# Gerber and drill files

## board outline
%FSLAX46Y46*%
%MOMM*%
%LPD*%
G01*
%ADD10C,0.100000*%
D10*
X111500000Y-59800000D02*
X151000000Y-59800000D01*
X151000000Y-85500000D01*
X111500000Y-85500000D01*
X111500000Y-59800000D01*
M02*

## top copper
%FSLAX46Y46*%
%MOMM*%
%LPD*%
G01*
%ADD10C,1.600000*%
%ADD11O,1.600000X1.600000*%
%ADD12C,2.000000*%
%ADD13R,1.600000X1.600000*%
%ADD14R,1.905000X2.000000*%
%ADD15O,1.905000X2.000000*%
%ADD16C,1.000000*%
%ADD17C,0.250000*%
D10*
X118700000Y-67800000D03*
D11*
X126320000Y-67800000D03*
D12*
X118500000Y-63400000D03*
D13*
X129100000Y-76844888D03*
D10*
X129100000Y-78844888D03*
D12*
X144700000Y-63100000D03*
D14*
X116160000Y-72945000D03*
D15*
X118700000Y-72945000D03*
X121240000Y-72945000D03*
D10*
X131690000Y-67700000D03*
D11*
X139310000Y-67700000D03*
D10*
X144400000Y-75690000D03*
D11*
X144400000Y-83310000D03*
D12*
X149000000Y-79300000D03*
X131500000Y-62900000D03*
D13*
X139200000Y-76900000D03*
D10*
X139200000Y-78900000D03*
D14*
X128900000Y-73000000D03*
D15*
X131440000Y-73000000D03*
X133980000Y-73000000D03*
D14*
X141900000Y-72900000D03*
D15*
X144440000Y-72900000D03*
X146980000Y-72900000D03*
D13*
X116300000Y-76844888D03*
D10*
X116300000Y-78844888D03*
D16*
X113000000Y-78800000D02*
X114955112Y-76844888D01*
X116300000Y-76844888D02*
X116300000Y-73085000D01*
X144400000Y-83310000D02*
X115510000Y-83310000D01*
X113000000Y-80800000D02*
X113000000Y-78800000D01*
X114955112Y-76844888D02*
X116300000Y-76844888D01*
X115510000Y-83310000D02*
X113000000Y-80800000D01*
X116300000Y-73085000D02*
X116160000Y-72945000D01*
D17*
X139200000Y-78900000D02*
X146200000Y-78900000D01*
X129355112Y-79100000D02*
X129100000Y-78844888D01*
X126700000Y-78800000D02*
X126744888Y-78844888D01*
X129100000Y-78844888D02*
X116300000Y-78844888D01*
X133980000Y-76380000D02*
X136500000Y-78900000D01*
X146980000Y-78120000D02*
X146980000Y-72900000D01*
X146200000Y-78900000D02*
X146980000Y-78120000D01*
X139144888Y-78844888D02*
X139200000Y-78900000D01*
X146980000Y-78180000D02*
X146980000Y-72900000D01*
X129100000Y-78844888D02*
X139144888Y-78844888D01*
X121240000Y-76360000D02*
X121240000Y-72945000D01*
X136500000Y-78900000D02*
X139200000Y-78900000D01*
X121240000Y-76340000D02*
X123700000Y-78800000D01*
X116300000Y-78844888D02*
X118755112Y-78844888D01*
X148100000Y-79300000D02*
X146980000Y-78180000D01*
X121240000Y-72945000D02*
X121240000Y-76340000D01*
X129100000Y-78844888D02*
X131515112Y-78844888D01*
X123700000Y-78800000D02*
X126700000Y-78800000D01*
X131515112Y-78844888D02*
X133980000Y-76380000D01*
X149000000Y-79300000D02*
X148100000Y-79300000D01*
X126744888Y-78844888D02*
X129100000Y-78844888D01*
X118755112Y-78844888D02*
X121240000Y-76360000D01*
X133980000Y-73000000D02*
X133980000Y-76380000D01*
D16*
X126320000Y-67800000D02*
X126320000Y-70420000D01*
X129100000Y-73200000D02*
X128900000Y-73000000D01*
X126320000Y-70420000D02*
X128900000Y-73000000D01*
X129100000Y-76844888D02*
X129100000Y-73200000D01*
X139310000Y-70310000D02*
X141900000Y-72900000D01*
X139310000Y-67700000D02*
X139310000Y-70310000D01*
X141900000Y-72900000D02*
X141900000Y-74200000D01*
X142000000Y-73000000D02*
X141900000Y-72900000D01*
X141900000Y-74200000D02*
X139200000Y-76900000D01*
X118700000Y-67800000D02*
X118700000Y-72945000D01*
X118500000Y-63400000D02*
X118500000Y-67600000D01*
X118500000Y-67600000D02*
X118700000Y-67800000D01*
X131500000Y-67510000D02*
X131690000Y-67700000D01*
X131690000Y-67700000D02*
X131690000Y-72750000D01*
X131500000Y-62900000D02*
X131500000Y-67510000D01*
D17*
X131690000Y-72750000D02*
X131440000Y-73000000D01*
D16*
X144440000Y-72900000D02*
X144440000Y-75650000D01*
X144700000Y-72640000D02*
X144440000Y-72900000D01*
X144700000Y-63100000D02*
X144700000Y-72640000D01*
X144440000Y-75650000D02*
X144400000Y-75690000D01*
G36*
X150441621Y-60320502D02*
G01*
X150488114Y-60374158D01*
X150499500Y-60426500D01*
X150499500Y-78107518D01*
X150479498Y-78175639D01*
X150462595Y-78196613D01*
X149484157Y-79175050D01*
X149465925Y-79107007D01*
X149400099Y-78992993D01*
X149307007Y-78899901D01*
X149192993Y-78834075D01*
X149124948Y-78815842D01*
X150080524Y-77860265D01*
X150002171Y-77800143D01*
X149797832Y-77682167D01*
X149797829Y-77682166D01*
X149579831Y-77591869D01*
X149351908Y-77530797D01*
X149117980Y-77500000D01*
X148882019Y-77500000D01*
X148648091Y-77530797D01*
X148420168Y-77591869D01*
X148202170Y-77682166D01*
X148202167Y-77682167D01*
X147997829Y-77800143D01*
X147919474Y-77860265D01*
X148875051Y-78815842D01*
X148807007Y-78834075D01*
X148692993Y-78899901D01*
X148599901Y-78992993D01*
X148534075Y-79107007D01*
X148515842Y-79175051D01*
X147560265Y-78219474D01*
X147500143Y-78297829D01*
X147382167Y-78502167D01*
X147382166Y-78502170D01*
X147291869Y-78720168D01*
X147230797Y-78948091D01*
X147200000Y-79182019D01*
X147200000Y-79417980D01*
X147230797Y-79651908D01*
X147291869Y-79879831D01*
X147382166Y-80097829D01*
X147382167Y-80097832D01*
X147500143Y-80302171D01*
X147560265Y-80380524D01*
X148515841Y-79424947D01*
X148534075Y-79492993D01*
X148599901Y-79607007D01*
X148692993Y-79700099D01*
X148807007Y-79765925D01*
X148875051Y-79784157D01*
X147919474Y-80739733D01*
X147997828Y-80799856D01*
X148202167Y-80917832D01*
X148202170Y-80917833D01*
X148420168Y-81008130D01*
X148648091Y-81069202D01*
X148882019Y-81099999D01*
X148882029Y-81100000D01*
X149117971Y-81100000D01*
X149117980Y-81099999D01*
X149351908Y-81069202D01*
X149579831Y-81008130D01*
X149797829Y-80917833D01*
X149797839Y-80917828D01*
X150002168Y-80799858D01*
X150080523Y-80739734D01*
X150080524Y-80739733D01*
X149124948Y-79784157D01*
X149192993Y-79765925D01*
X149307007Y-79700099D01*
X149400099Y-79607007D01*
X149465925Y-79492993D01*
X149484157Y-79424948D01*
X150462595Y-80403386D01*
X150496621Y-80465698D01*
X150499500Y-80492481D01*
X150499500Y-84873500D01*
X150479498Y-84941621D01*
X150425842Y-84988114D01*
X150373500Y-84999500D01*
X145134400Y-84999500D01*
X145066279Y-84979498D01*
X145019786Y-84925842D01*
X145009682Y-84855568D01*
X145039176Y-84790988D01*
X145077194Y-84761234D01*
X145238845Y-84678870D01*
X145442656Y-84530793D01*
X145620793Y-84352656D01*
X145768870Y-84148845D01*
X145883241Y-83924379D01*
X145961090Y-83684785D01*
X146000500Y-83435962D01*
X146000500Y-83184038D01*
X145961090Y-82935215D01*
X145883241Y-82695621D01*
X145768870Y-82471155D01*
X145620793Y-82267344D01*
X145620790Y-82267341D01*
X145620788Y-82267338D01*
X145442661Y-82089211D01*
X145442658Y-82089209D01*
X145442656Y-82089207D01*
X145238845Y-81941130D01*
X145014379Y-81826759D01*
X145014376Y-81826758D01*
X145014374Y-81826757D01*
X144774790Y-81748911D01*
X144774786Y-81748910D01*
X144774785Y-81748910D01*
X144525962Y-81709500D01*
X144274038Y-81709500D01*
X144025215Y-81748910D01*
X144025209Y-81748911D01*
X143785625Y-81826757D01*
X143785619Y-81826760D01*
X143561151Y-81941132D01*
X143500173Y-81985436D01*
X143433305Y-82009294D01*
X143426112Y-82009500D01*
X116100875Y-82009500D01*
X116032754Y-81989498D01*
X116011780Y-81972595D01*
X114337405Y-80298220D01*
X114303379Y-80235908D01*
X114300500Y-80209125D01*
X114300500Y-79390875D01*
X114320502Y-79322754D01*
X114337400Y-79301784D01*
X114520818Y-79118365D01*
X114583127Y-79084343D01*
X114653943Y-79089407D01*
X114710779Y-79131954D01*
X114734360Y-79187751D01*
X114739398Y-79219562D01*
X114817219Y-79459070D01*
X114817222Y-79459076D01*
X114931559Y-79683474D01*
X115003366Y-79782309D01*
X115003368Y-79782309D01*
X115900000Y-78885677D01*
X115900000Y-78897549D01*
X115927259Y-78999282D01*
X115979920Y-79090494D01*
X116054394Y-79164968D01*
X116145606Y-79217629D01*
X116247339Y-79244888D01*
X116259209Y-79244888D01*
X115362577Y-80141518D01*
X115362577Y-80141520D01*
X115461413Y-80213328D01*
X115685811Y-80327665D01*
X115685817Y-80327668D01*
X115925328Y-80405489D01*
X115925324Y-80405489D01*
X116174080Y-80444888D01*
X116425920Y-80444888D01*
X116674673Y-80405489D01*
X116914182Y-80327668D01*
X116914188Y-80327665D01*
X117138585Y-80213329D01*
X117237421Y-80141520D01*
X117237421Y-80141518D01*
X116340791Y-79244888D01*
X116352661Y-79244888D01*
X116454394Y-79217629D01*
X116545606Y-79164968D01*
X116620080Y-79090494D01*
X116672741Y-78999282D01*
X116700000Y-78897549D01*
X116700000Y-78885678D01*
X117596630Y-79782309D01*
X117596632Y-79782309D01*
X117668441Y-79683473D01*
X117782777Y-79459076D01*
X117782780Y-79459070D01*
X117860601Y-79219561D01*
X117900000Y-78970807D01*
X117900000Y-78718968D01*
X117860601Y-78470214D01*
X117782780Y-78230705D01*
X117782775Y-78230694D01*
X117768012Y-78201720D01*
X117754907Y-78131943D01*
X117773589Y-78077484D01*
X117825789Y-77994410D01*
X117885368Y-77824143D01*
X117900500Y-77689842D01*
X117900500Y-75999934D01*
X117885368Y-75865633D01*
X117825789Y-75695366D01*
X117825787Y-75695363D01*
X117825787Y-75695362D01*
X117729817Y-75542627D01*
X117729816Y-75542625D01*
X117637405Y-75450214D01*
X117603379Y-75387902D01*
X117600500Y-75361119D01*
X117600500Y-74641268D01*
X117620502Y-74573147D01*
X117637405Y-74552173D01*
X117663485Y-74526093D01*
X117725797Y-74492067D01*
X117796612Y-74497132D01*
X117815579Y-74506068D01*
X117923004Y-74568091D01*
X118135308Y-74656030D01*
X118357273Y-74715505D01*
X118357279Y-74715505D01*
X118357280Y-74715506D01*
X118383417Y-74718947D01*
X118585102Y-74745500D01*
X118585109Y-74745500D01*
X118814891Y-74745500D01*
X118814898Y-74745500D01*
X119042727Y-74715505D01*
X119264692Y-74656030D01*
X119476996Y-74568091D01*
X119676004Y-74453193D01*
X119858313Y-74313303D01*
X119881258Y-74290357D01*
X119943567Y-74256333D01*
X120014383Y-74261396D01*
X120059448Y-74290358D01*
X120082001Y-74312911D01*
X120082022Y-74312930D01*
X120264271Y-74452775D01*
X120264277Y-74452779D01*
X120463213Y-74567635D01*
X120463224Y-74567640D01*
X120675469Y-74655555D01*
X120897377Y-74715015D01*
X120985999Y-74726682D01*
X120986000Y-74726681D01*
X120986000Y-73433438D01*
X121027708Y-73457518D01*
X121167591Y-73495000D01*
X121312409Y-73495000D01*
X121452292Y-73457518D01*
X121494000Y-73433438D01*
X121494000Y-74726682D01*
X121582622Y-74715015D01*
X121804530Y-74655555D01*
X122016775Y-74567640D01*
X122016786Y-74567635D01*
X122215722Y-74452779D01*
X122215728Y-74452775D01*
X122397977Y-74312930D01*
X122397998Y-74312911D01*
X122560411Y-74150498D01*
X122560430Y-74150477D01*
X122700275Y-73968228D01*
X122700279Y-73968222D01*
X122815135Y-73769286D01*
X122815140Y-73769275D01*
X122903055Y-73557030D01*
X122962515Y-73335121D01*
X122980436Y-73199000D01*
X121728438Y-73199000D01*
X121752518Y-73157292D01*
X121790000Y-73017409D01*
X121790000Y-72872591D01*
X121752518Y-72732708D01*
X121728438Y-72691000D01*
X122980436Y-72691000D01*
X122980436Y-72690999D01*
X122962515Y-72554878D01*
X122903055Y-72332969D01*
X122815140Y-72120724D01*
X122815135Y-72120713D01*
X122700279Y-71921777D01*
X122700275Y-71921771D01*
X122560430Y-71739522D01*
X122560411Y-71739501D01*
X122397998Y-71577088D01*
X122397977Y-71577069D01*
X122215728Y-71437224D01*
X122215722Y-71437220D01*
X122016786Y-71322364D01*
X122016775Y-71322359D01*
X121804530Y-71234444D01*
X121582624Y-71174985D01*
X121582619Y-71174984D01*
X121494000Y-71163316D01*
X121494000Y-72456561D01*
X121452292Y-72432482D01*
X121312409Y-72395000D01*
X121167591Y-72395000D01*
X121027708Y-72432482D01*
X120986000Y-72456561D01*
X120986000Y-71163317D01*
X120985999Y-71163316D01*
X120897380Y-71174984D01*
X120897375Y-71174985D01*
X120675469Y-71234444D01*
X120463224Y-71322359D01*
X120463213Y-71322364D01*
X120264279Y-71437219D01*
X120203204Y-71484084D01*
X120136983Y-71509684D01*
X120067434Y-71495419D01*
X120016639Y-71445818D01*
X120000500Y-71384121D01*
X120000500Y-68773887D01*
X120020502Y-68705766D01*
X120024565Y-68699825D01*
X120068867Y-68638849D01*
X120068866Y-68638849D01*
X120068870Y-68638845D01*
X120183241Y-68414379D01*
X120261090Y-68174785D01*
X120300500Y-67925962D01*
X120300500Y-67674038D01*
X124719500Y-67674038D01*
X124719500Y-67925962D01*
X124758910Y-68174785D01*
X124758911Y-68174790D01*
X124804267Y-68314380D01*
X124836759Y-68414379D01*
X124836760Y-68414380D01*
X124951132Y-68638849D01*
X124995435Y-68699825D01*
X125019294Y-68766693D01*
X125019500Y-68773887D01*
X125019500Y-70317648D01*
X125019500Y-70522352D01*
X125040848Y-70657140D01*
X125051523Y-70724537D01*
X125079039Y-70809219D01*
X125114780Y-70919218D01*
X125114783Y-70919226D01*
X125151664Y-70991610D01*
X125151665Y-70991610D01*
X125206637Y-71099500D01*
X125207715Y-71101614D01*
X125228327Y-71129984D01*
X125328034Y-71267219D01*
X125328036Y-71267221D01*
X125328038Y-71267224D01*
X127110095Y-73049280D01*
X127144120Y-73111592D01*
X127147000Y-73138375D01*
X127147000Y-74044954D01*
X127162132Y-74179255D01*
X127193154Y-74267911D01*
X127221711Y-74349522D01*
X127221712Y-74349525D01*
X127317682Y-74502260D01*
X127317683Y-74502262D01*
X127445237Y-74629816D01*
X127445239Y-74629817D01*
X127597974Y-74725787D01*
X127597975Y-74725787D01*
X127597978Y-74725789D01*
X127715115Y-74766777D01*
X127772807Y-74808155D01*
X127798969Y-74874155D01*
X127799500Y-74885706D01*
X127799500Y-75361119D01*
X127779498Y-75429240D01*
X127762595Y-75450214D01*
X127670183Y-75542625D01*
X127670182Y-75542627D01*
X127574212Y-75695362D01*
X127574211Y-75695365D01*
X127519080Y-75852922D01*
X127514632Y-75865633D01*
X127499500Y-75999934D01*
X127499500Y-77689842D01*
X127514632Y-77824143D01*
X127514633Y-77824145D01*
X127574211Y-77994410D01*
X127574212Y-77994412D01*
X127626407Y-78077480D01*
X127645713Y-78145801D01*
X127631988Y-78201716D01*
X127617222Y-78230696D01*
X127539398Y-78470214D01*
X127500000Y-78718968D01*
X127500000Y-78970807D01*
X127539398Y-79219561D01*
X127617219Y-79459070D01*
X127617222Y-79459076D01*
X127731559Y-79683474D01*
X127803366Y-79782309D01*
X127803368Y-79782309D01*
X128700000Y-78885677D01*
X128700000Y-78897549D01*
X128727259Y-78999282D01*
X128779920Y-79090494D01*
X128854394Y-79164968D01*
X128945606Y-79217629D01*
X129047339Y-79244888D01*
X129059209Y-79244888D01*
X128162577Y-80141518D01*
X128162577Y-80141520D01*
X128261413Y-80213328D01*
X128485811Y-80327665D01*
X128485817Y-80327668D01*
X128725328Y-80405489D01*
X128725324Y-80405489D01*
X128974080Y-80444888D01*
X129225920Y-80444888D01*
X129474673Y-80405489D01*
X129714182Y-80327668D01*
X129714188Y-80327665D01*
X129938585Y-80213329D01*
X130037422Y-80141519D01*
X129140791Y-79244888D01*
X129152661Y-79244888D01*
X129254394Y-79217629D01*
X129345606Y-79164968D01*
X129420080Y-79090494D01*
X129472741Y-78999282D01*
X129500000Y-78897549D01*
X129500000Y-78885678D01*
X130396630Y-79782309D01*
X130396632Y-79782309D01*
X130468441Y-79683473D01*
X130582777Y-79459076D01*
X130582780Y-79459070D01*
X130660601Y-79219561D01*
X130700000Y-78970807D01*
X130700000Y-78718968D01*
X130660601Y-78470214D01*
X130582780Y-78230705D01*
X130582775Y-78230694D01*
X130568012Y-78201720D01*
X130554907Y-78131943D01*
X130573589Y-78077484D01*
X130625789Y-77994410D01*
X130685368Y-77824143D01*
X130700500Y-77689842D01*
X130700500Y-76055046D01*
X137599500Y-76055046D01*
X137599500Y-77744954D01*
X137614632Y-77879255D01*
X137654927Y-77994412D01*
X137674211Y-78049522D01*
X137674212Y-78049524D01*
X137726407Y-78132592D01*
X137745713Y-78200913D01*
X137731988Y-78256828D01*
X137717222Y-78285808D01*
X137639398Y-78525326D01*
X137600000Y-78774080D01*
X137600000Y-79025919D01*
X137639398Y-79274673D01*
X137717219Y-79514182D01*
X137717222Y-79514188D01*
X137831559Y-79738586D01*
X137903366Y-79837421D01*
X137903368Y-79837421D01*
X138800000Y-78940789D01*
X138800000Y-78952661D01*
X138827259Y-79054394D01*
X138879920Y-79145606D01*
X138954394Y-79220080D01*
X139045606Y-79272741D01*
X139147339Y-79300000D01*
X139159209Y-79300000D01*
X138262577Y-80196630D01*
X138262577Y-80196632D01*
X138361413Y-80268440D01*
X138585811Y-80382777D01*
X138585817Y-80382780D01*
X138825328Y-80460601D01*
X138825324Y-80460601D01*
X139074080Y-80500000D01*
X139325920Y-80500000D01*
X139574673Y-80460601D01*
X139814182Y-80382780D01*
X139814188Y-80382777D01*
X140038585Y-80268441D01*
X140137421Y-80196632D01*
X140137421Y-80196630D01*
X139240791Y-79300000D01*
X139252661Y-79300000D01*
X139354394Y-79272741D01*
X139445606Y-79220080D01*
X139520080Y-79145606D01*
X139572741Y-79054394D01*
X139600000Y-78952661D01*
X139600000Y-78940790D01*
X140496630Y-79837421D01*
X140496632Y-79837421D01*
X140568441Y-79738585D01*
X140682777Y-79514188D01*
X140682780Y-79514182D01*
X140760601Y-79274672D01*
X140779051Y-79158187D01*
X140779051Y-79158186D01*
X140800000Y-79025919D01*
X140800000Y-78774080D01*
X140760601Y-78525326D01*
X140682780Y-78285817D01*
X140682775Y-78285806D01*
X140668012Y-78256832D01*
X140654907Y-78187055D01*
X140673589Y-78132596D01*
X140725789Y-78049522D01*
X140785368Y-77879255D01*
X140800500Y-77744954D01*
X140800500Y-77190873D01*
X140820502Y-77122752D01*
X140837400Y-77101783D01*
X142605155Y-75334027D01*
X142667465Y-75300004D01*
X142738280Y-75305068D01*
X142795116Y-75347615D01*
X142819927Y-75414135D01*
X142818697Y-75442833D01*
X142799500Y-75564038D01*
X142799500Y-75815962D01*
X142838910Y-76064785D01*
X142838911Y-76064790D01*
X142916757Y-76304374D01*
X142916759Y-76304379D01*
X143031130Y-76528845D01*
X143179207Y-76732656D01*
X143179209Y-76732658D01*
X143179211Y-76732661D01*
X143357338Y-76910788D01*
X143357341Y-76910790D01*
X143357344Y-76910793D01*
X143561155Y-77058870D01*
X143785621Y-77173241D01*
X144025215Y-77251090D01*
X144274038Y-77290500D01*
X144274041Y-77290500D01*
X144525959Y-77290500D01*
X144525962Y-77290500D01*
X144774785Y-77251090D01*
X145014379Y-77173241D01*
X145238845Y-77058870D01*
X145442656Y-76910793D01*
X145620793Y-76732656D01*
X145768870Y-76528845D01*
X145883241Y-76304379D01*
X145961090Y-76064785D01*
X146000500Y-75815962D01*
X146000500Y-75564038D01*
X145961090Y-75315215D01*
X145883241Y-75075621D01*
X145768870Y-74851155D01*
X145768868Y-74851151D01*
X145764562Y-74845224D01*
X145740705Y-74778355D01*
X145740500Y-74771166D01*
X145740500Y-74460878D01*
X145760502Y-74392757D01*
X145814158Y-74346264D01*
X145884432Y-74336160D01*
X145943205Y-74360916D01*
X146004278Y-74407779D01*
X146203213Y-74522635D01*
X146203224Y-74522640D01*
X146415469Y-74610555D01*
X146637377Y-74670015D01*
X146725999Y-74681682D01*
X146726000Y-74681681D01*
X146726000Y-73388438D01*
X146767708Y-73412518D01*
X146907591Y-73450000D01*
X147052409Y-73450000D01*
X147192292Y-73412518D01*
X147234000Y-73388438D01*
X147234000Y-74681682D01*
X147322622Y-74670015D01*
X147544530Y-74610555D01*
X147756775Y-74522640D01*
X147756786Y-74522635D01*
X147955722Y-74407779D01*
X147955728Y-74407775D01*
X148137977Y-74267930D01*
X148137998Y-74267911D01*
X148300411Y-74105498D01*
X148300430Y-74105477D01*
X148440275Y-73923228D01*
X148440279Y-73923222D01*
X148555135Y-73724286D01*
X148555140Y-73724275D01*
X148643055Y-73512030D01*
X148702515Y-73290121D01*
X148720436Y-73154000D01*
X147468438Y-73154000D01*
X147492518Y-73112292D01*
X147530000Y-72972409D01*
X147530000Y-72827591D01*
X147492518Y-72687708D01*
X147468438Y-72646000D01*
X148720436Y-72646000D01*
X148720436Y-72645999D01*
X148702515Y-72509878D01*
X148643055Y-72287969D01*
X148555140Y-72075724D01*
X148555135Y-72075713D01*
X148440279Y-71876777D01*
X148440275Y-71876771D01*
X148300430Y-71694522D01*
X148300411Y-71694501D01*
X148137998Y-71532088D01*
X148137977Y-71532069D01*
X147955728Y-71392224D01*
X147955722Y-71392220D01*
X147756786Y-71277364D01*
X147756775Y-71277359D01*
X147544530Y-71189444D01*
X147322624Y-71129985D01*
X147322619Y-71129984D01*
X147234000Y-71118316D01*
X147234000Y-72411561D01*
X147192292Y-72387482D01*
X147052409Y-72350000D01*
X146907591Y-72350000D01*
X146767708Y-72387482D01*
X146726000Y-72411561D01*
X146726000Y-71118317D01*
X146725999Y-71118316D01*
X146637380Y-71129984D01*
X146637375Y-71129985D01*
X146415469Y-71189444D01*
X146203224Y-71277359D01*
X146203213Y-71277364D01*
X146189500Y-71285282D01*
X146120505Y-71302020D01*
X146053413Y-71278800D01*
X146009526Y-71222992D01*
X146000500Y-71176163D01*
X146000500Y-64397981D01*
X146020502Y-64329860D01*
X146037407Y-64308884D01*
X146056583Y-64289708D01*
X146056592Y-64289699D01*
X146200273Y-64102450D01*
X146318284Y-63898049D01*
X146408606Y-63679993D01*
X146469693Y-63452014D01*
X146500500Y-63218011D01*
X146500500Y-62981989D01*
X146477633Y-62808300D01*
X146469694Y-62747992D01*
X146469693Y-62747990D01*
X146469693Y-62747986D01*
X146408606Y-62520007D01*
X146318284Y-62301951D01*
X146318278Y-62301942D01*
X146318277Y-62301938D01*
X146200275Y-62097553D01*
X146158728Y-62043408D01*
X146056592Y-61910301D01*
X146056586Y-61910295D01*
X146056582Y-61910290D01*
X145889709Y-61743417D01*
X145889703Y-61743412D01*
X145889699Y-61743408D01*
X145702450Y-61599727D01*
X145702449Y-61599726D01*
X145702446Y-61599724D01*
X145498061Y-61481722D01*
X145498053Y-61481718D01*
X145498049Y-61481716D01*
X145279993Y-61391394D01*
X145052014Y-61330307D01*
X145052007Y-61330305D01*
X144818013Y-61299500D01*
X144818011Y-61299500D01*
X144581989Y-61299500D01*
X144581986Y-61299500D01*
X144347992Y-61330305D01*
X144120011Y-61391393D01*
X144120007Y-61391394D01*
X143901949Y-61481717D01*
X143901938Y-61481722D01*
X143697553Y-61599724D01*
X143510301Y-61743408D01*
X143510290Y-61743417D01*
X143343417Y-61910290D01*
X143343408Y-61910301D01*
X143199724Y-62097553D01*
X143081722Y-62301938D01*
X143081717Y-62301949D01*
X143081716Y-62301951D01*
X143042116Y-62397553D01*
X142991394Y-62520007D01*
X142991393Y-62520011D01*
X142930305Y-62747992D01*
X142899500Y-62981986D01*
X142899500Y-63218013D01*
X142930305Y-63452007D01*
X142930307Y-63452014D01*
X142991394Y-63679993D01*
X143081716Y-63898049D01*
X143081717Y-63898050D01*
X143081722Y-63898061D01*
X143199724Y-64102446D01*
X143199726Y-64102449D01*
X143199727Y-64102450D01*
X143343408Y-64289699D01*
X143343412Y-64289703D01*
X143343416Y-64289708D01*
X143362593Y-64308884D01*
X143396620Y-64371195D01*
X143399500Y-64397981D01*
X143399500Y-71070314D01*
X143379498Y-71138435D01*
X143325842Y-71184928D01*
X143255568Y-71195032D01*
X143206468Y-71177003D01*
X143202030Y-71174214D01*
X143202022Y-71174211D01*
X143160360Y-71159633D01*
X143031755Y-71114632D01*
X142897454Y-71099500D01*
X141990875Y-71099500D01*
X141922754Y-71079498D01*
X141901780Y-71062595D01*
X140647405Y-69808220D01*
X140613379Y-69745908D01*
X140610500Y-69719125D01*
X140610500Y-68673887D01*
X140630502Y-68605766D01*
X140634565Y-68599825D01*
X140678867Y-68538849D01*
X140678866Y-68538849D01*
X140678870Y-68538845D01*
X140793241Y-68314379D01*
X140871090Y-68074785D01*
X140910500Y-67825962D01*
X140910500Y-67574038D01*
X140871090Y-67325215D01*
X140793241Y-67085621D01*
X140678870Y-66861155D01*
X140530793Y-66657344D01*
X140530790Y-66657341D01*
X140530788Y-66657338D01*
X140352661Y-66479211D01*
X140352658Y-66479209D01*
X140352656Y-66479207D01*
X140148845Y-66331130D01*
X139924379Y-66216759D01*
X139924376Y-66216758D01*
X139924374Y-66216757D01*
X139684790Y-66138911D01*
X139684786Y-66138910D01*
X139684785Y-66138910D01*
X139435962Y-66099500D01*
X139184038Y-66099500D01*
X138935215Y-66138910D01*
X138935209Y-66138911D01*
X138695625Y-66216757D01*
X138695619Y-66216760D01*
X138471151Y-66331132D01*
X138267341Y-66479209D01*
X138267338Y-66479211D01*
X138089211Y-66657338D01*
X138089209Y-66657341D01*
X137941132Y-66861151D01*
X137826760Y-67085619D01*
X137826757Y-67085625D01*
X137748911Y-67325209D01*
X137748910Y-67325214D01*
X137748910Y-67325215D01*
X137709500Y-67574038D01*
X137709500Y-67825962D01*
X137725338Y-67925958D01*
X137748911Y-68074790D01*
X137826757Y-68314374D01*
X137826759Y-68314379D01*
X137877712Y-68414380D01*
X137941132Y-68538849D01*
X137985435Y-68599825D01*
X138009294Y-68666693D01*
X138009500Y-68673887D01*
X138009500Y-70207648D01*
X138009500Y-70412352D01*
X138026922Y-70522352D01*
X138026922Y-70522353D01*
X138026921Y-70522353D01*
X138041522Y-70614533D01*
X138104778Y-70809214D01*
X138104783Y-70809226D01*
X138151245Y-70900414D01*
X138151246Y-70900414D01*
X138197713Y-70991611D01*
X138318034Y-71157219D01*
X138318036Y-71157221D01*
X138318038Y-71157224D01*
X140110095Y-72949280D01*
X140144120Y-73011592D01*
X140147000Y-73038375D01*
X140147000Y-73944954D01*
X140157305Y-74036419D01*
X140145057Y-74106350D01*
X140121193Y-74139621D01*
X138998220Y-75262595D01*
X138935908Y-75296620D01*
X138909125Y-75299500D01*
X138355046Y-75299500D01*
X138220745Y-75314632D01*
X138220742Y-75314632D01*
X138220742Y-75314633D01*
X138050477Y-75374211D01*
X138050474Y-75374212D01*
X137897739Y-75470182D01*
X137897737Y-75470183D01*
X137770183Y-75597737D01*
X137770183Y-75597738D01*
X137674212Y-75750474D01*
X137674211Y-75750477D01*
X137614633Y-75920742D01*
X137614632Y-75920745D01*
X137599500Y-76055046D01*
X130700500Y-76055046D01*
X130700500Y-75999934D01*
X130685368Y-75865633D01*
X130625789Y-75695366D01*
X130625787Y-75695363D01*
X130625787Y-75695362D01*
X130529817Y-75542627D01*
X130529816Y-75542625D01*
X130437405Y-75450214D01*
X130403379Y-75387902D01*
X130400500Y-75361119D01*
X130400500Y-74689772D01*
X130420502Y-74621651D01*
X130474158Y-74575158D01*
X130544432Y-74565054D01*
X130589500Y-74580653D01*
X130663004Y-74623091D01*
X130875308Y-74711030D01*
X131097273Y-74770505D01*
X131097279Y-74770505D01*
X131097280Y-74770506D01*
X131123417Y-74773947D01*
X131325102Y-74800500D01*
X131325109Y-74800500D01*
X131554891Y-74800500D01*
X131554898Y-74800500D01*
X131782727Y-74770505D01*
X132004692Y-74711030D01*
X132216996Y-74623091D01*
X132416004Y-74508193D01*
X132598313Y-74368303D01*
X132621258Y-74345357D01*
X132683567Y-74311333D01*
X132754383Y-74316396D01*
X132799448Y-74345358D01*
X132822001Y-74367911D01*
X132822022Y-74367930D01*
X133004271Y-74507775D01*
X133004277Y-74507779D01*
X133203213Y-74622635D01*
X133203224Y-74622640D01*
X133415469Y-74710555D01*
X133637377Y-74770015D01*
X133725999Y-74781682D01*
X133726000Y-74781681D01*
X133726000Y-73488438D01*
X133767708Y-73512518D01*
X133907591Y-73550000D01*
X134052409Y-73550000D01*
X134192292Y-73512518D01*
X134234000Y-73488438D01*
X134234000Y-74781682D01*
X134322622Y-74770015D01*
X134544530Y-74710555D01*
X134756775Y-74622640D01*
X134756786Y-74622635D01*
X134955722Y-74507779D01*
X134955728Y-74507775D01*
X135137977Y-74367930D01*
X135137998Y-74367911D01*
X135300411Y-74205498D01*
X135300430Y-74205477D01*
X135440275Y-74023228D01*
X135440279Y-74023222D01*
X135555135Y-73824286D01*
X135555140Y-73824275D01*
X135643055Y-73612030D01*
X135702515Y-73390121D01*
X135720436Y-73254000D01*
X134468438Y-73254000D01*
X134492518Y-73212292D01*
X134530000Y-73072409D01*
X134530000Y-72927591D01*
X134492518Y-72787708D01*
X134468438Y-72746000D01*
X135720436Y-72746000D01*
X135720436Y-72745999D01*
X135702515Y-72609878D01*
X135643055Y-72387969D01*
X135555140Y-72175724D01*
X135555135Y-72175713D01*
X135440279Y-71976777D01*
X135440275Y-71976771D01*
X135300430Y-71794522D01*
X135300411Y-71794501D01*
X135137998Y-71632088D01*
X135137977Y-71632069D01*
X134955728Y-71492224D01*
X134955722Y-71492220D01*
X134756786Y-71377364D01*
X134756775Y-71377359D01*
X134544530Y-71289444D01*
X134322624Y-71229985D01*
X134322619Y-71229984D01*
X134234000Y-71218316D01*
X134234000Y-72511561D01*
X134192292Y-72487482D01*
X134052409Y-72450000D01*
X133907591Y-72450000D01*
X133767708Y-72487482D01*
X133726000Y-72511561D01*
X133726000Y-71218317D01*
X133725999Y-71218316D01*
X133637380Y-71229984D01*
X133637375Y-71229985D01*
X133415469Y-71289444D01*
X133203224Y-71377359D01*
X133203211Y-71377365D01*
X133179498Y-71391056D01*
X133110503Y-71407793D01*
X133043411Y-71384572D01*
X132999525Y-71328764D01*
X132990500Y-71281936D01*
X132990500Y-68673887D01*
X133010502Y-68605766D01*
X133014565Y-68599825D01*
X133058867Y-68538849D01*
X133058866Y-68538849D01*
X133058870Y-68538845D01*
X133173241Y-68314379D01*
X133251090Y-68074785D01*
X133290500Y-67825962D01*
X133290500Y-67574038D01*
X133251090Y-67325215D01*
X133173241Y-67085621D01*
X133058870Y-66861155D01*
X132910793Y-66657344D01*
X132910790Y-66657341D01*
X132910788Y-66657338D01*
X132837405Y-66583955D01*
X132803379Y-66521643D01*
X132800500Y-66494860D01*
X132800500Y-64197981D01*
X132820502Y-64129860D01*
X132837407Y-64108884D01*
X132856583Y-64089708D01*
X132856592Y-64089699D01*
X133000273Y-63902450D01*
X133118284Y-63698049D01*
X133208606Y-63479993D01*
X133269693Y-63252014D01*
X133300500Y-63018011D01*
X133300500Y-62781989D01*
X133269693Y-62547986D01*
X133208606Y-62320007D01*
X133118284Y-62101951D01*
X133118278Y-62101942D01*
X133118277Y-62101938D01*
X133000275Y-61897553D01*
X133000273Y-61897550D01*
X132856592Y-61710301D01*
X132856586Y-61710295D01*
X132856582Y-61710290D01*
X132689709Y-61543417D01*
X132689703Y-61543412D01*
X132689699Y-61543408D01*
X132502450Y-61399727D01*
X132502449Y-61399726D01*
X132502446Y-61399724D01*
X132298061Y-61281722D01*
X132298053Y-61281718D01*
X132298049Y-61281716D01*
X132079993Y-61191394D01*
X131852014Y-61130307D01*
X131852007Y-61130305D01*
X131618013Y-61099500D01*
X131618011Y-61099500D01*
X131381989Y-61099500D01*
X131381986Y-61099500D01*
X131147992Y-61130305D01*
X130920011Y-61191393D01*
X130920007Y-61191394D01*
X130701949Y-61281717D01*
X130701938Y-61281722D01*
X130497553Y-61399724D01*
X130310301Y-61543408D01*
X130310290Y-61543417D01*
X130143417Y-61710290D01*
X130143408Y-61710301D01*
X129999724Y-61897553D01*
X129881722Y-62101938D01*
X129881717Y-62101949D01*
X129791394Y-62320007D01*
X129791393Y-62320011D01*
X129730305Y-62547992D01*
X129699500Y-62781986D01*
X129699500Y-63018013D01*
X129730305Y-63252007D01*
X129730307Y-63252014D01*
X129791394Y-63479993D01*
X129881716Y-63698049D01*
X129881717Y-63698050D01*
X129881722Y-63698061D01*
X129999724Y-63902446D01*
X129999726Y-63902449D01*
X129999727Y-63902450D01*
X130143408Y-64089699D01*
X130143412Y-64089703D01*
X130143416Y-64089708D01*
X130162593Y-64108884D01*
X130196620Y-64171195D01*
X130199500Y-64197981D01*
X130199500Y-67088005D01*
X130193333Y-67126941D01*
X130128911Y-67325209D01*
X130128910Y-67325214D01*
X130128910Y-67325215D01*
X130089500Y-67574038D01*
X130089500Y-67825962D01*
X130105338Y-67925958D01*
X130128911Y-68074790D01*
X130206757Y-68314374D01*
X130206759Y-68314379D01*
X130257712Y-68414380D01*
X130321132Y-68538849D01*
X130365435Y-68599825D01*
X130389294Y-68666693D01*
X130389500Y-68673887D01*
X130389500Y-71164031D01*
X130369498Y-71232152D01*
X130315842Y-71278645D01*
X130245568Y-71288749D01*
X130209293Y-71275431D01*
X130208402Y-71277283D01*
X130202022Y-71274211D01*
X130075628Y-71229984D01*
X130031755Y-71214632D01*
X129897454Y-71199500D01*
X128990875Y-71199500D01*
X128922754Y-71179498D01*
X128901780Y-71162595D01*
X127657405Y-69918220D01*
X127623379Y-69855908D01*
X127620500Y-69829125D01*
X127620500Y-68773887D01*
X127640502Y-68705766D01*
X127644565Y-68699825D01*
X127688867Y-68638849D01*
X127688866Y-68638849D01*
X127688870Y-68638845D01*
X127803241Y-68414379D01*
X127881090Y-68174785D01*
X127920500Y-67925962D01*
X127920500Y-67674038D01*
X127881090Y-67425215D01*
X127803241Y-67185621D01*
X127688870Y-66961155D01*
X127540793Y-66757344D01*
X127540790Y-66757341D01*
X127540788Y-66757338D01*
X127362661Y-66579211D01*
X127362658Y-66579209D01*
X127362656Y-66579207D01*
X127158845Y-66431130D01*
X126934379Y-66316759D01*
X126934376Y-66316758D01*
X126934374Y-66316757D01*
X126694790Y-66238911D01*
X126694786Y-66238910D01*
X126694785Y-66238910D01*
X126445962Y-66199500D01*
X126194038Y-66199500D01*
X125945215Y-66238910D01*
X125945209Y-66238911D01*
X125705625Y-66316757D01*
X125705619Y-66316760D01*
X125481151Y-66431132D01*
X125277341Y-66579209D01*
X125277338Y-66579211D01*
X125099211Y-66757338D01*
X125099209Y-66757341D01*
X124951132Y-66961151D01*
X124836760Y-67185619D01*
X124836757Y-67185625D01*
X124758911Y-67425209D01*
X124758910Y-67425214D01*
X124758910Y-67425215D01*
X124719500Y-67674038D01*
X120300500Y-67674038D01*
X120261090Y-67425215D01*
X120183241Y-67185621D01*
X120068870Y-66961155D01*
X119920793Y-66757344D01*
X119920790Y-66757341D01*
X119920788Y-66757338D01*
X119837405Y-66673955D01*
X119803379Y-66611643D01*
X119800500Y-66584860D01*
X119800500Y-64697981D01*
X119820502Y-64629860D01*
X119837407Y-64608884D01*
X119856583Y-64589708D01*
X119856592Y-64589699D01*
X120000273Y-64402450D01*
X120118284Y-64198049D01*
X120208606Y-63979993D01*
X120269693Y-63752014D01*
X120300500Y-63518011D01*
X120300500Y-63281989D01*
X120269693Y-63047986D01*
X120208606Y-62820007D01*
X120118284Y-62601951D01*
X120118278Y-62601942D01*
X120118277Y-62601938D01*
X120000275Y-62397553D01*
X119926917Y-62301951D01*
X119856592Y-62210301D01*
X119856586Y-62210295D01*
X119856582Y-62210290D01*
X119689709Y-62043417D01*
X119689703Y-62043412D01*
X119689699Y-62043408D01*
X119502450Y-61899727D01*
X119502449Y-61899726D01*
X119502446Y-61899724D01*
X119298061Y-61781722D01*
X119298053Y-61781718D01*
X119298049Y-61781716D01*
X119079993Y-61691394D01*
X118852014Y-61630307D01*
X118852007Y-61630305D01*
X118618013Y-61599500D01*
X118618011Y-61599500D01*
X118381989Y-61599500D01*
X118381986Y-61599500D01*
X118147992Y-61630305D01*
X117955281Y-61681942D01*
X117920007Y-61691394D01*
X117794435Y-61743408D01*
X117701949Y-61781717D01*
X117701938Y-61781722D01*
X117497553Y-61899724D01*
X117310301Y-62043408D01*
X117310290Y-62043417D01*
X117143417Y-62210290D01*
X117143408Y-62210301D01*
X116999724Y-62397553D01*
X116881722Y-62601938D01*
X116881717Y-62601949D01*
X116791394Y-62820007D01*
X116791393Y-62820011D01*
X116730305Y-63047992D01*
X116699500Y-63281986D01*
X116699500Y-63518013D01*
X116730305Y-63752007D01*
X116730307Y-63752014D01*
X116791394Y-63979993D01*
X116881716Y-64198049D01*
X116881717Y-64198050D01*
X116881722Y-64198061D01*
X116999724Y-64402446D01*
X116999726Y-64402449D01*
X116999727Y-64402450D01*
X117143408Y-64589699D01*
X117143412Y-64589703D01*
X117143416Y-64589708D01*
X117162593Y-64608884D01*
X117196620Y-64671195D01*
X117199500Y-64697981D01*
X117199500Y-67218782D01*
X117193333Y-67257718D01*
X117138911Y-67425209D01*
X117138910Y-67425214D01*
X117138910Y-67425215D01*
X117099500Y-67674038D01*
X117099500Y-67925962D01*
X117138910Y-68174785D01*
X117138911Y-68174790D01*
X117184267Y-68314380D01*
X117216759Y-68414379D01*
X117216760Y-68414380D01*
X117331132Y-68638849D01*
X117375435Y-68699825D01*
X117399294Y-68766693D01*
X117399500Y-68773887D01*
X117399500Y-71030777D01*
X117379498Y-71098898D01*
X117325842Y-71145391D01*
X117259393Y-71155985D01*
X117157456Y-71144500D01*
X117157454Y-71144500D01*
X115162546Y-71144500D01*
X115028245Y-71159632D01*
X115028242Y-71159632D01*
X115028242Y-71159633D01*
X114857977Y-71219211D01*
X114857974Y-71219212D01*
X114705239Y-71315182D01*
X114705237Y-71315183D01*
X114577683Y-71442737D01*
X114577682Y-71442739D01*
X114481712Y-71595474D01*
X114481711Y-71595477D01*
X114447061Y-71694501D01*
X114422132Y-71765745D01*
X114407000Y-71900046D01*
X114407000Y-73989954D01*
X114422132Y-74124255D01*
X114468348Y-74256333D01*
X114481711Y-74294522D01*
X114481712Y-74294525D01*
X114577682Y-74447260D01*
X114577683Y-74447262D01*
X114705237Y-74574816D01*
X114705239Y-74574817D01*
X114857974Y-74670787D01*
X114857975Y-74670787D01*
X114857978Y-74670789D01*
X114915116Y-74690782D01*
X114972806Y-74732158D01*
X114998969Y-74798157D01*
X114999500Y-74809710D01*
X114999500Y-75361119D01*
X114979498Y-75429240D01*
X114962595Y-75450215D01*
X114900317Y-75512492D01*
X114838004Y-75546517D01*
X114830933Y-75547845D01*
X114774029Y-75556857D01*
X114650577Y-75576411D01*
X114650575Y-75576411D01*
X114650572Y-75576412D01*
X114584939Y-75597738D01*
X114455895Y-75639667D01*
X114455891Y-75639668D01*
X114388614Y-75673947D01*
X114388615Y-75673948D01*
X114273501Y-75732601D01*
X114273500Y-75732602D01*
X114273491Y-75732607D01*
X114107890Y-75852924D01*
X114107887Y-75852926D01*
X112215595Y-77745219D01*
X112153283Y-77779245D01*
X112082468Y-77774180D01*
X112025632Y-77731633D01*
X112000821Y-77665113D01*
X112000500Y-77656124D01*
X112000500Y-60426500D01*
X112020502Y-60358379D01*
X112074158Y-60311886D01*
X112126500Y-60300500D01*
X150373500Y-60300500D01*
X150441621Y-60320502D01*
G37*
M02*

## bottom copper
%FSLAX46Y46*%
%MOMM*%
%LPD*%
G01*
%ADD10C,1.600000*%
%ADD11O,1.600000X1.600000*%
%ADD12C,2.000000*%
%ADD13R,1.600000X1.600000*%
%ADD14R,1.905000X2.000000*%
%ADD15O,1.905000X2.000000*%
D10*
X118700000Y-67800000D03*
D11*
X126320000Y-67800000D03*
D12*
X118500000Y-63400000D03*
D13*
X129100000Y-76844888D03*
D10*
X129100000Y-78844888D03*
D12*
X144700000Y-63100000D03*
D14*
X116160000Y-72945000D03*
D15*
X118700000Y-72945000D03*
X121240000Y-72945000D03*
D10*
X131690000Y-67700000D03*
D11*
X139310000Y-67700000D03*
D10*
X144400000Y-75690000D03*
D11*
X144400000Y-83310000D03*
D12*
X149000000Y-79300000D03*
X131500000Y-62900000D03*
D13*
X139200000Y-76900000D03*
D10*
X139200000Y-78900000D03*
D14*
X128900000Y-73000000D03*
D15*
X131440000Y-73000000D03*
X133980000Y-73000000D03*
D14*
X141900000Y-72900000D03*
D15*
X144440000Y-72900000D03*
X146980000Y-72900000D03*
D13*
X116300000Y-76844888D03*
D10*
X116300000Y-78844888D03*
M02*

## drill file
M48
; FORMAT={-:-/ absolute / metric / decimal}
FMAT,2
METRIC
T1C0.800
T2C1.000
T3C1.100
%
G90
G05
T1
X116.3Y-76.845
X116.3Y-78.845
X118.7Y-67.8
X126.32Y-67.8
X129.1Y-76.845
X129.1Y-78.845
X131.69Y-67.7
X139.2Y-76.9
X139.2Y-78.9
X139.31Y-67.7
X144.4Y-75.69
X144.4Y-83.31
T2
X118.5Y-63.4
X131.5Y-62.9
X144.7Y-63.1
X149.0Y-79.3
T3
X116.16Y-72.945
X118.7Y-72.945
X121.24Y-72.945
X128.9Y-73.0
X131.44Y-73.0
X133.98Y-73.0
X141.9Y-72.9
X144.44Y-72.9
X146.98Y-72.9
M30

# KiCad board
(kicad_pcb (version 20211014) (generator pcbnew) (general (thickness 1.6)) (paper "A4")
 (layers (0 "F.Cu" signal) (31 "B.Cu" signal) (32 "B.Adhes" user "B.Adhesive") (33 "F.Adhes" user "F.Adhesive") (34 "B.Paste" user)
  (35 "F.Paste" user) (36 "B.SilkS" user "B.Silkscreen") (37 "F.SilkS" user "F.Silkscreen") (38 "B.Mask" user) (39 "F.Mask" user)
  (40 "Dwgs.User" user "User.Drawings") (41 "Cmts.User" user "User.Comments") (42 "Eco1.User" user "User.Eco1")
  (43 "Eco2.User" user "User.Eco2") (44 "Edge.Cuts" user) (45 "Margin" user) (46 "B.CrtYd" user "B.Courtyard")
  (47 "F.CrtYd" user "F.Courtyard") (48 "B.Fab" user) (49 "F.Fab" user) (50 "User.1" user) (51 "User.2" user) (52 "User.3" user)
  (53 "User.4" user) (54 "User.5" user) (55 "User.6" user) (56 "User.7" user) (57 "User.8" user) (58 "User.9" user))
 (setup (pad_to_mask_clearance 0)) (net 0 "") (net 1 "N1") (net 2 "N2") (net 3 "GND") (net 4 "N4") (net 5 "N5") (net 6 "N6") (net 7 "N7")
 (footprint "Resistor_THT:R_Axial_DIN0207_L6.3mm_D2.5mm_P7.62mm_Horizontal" (layer "F.Cu") (at 118.7 67.8)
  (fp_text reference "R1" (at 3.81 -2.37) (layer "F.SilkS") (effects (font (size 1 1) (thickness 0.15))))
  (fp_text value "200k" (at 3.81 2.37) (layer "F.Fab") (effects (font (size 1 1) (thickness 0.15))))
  (pad "1" thru_hole circle (at 0 0) (size 1.6 1.6) (drill 0.8) (layers *.Cu *.Mask) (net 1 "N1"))
  (pad "2" thru_hole oval (at 7.62 0) (size 1.6 1.6) (drill 0.8) (layers *.Cu *.Mask) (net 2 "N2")))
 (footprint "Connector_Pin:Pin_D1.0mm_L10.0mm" (layer "F.Cu") (at 118.5 63.4)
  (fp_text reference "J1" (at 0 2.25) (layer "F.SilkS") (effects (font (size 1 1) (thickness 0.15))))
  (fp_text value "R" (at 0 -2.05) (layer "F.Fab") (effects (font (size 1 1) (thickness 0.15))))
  (pad "1" thru_hole circle (at 0 0) (size 2 2) (drill 1) (layers *.Cu *.Mask) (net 1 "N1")))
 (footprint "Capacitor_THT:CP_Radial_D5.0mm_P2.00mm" (layer "F.Cu") (at 129.1 76.844888 -90)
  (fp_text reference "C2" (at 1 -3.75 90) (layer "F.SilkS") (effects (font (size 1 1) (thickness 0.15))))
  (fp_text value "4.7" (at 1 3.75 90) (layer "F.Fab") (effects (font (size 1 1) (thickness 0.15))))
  (pad "1" thru_hole rect (at 0 0 270) (size 1.6 1.6) (drill 0.8) (layers *.Cu *.Mask) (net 2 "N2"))
  (pad "2" thru_hole circle (at 2 0 270) (size 1.6 1.6) (drill 0.8) (layers *.Cu *.Mask) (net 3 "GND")))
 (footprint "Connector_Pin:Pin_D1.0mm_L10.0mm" (layer "F.Cu") (at 144.7 63.1)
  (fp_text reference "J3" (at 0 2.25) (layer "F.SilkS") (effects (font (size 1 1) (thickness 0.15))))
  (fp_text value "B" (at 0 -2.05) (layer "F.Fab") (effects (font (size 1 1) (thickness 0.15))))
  (pad "1" thru_hole circle (at 0 0) (size 2 2) (drill 1) (layers *.Cu *.Mask) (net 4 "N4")))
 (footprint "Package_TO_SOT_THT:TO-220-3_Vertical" (layer "F.Cu") (at 116.16 72.945)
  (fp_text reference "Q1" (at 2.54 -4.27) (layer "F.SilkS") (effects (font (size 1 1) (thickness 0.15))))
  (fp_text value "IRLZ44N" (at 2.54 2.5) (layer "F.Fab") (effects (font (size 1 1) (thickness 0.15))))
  (pad "1" thru_hole rect (at 0 0) (size 1.905 2) (drill 1.1) (layers *.Cu *.Mask) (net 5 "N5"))
  (pad "2" thru_hole oval (at 2.54 0) (size 1.905 2) (drill 1.1) (layers *.Cu *.Mask) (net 1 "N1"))
  (pad "3" thru_hole oval (at 5.08 0) (size 1.905 2) (drill 1.1) (layers *.Cu *.Mask) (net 3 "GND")))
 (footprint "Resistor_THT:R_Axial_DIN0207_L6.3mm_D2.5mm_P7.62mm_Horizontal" (layer "F.Cu") (at 131.69 67.7)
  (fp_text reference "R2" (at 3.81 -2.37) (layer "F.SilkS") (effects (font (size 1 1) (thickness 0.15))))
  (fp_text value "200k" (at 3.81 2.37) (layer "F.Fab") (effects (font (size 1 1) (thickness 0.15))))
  (pad "1" thru_hole circle (at 0 0) (size 1.6 1.6) (drill 0.8) (layers *.Cu *.Mask) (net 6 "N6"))
  (pad "2" thru_hole oval (at 7.62 0) (size 1.6 1.6) (drill 0.8) (layers *.Cu *.Mask) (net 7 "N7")))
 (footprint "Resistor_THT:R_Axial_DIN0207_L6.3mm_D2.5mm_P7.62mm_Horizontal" (layer "F.Cu") (at 144.4 75.69 -90)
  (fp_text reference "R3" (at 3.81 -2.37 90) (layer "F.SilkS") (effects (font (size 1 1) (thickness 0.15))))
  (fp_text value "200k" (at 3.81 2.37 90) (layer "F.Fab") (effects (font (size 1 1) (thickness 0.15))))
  (pad "1" thru_hole circle (at 0 0 270) (size 1.6 1.6) (drill 0.8) (layers *.Cu *.Mask) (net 4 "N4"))
  (pad "2" thru_hole oval (at 7.62 0 270) (size 1.6 1.6) (drill 0.8) (layers *.Cu *.Mask) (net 5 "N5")))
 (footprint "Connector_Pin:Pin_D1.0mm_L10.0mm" (layer "F.Cu") (at 149 79.3)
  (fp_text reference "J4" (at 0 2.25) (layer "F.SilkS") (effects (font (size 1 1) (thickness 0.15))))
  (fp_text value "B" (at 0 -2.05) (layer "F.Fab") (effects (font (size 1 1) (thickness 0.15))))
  (pad "1" thru_hole circle (at 0 0) (size 2 2) (drill 1) (layers *.Cu *.Mask) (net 3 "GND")))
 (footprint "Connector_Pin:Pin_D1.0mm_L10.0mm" (layer "F.Cu") (at 131.5 62.9)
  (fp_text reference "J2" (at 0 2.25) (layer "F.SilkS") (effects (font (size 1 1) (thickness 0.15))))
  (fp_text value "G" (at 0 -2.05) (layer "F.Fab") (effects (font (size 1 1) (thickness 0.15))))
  (pad "1" thru_hole circle (at 0 0) (size 2 2) (drill 1) (layers *.Cu *.Mask) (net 6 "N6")))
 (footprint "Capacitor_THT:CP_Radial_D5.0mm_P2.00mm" (layer "F.Cu") (at 139.2 76.9 -90)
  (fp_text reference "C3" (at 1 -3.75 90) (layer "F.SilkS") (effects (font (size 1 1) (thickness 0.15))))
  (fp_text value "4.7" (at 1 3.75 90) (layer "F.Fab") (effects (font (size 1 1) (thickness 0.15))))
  (pad "1" thru_hole rect (at 0 0 270) (size 1.6 1.6) (drill 0.8) (layers *.Cu *.Mask) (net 7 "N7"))
  (pad "2" thru_hole circle (at 2 0 270) (size 1.6 1.6) (drill 0.8) (layers *.Cu *.Mask) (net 3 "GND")))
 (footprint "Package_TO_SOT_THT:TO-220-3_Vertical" (layer "F.Cu") (at 128.9 73)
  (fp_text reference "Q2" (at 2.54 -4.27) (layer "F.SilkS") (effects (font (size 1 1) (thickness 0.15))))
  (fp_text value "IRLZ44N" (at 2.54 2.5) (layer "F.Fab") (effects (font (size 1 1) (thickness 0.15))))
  (pad "1" thru_hole rect (at 0 0) (size 1.905 2) (drill 1.1) (layers *.Cu *.Mask) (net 2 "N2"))
  (pad "2" thru_hole oval (at 2.54 0) (size 1.905 2) (drill 1.1) (layers *.Cu *.Mask) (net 6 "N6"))
  (pad "3" thru_hole oval (at 5.08 0) (size 1.905 2) (drill 1.1) (layers *.Cu *.Mask) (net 3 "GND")))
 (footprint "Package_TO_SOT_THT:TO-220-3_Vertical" (layer "F.Cu") (at 141.9 72.9)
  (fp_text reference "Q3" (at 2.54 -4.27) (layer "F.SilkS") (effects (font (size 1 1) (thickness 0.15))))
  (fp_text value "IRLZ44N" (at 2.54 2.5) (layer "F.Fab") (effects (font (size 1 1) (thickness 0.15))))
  (pad "1" thru_hole rect (at 0 0) (size 1.905 2) (drill 1.1) (layers *.Cu *.Mask) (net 7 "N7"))
  (pad "2" thru_hole oval (at 2.54 0) (size 1.905 2) (drill 1.1) (layers *.Cu *.Mask) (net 4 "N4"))
  (pad "3" thru_hole oval (at 5.08 0) (size 1.905 2) (drill 1.1) (layers *.Cu *.Mask) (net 3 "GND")))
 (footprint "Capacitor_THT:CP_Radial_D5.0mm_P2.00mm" (layer "F.Cu") (at 116.3 76.844888 -90)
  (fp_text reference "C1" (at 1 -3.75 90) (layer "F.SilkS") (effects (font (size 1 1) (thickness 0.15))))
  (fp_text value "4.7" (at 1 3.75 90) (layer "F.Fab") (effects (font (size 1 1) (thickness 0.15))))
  (pad "1" thru_hole rect (at 0 0 270) (size 1.6 1.6) (drill 0.8) (layers *.Cu *.Mask) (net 5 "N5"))
  (pad "2" thru_hole circle (at 2 0 270) (size 1.6 1.6) (drill 0.8) (layers *.Cu *.Mask) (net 3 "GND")))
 (gr_rect (start 151 85.5) (end 111.5 59.8) (layer "Edge.Cuts") (width 0.1) (fill none))
 (segment (start 113 78.8) (end 114.955112 76.844888) (width 1) (layer "F.Cu") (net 5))
 (segment (start 116.3 76.844888) (end 116.3 73.085) (width 1) (layer "F.Cu") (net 5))
 (segment (start 144.4 83.31) (end 115.51 83.31) (width 1) (layer "F.Cu") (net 5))
 (segment (start 113 80.8) (end 113 78.8) (width 1) (layer "F.Cu") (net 5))
 (segment (start 114.955112 76.844888) (end 116.3 76.844888) (width 1) (layer "F.Cu") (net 5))
 (segment (start 115.51 83.31) (end 113 80.8) (width 1) (layer "F.Cu") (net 5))
 (segment (start 116.3 73.085) (end 116.16 72.945) (width 1) (layer "F.Cu") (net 5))
 (segment (start 139.2 78.9) (end 146.2 78.9) (width 0.25) (layer "F.Cu") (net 3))
 (segment (start 129.355112 79.1) (end 129.1 78.844888) (width 0.25) (layer "F.Cu") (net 3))
 (segment (start 126.7 78.8) (end 126.744888 78.844888) (width 0.25) (layer "F.Cu") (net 3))
 (segment (start 129.1 78.844888) (end 116.3 78.844888) (width 0.25) (layer "F.Cu") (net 3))
 (segment (start 133.98 76.38) (end 136.5 78.9) (width 0.25) (layer "F.Cu") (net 3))
 (segment (start 146.98 78.12) (end 146.98 72.9) (width 0.25) (layer "F.Cu") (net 3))
 (segment (start 146.2 78.9) (end 146.98 78.12) (width 0.25) (layer "F.Cu") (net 3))
 (segment (start 139.144888 78.844888) (end 139.2 78.9) (width 0.25) (layer "F.Cu") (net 3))
 (segment (start 146.98 78.18) (end 146.98 72.9) (width 0.25) (layer "F.Cu") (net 3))
 (segment (start 129.1 78.844888) (end 139.144888 78.844888) (width 0.25) (layer "F.Cu") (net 3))
 (segment (start 121.24 76.36) (end 121.24 72.945) (width 0.25) (layer "F.Cu") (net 3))
 (segment (start 136.5 78.9) (end 139.2 78.9) (width 0.25) (layer "F.Cu") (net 3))
 (segment (start 121.24 76.34) (end 123.7 78.8) (width 0.25) (layer "F.Cu") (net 3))
 (segment (start 116.3 78.844888) (end 118.755112 78.844888) (width 0.25) (layer "F.Cu") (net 3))
 (segment (start 148.1 79.3) (end 146.98 78.18) (width 0.25) (layer "F.Cu") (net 3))
 (segment (start 121.24 72.945) (end 121.24 76.34) (width 0.25) (layer "F.Cu") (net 3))
 (segment (start 129.1 78.844888) (end 131.515112 78.844888) (width 0.25) (layer "F.Cu") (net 3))
 (segment (start 123.7 78.8) (end 126.7 78.8) (width 0.25) (layer "F.Cu") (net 3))
 (segment (start 131.515112 78.844888) (end 133.98 76.38) (width 0.25) (layer "F.Cu") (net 3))
 (segment (start 149 79.3) (end 148.1 79.3) (width 0.25) (layer "F.Cu") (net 3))
 (segment (start 126.744888 78.844888) (end 129.1 78.844888) (width 0.25) (layer "F.Cu") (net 3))
 (segment (start 118.755112 78.844888) (end 121.24 76.36) (width 0.25) (layer "F.Cu") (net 3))
 (segment (start 133.98 73) (end 133.98 76.38) (width 0.25) (layer "F.Cu") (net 3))
 (segment (start 126.32 67.8) (end 126.32 70.42) (width 1) (layer "F.Cu") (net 2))
 (segment (start 129.1 73.2) (end 128.9 73) (width 1) (layer "F.Cu") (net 2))
 (segment (start 126.32 70.42) (end 128.9 73) (width 1) (layer "F.Cu") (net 2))
 (segment (start 129.1 76.844888) (end 129.1 73.2) (width 1) (layer "F.Cu") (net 2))
 (segment (start 139.31 70.31) (end 141.9 72.9) (width 1) (layer "F.Cu") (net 7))
 (segment (start 139.31 67.7) (end 139.31 70.31) (width 1) (layer "F.Cu") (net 7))
 (segment (start 141.9 72.9) (end 141.9 74.2) (width 1) (layer "F.Cu") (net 7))
 (segment (start 142 73) (end 141.9 72.9) (width 1) (layer "F.Cu") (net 7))
 (segment (start 141.9 74.2) (end 139.2 76.9) (width 1) (layer "F.Cu") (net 7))
 (segment (start 118.7 67.8) (end 118.7 72.945) (width 1) (layer "F.Cu") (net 1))
 (segment (start 118.5 63.4) (end 118.5 67.6) (width 1) (layer "F.Cu") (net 1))
 (segment (start 118.5 67.6) (end 118.7 67.8) (width 1) (layer "F.Cu") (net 1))
 (segment (start 131.5 67.51) (end 131.69 67.7) (width 1) (layer "F.Cu") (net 6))
 (segment (start 131.69 67.7) (end 131.69 72.75) (width 1) (layer "F.Cu") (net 6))
 (segment (start 131.5 62.9) (end 131.5 67.51) (width 1) (layer "F.Cu") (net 6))
 (segment (start 131.69 72.75) (end 131.44 73) (width 0.25) (layer "F.Cu") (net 6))
 (segment (start 144.44 72.9) (end 144.44 75.65) (width 1) (layer "F.Cu") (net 4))
 (segment (start 144.7 72.64) (end 144.44 72.9) (width 1) (layer "F.Cu") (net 4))
 (segment (start 144.7 63.1) (end 144.7 72.64) (width 1) (layer "F.Cu") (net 4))
 (segment (start 144.44 75.65) (end 144.4 75.69) (width 1) (layer "F.Cu") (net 4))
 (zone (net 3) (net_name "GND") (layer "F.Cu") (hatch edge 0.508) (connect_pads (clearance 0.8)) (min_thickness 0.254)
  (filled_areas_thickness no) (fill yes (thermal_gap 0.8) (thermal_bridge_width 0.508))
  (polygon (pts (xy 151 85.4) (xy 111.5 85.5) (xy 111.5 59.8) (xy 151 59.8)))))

